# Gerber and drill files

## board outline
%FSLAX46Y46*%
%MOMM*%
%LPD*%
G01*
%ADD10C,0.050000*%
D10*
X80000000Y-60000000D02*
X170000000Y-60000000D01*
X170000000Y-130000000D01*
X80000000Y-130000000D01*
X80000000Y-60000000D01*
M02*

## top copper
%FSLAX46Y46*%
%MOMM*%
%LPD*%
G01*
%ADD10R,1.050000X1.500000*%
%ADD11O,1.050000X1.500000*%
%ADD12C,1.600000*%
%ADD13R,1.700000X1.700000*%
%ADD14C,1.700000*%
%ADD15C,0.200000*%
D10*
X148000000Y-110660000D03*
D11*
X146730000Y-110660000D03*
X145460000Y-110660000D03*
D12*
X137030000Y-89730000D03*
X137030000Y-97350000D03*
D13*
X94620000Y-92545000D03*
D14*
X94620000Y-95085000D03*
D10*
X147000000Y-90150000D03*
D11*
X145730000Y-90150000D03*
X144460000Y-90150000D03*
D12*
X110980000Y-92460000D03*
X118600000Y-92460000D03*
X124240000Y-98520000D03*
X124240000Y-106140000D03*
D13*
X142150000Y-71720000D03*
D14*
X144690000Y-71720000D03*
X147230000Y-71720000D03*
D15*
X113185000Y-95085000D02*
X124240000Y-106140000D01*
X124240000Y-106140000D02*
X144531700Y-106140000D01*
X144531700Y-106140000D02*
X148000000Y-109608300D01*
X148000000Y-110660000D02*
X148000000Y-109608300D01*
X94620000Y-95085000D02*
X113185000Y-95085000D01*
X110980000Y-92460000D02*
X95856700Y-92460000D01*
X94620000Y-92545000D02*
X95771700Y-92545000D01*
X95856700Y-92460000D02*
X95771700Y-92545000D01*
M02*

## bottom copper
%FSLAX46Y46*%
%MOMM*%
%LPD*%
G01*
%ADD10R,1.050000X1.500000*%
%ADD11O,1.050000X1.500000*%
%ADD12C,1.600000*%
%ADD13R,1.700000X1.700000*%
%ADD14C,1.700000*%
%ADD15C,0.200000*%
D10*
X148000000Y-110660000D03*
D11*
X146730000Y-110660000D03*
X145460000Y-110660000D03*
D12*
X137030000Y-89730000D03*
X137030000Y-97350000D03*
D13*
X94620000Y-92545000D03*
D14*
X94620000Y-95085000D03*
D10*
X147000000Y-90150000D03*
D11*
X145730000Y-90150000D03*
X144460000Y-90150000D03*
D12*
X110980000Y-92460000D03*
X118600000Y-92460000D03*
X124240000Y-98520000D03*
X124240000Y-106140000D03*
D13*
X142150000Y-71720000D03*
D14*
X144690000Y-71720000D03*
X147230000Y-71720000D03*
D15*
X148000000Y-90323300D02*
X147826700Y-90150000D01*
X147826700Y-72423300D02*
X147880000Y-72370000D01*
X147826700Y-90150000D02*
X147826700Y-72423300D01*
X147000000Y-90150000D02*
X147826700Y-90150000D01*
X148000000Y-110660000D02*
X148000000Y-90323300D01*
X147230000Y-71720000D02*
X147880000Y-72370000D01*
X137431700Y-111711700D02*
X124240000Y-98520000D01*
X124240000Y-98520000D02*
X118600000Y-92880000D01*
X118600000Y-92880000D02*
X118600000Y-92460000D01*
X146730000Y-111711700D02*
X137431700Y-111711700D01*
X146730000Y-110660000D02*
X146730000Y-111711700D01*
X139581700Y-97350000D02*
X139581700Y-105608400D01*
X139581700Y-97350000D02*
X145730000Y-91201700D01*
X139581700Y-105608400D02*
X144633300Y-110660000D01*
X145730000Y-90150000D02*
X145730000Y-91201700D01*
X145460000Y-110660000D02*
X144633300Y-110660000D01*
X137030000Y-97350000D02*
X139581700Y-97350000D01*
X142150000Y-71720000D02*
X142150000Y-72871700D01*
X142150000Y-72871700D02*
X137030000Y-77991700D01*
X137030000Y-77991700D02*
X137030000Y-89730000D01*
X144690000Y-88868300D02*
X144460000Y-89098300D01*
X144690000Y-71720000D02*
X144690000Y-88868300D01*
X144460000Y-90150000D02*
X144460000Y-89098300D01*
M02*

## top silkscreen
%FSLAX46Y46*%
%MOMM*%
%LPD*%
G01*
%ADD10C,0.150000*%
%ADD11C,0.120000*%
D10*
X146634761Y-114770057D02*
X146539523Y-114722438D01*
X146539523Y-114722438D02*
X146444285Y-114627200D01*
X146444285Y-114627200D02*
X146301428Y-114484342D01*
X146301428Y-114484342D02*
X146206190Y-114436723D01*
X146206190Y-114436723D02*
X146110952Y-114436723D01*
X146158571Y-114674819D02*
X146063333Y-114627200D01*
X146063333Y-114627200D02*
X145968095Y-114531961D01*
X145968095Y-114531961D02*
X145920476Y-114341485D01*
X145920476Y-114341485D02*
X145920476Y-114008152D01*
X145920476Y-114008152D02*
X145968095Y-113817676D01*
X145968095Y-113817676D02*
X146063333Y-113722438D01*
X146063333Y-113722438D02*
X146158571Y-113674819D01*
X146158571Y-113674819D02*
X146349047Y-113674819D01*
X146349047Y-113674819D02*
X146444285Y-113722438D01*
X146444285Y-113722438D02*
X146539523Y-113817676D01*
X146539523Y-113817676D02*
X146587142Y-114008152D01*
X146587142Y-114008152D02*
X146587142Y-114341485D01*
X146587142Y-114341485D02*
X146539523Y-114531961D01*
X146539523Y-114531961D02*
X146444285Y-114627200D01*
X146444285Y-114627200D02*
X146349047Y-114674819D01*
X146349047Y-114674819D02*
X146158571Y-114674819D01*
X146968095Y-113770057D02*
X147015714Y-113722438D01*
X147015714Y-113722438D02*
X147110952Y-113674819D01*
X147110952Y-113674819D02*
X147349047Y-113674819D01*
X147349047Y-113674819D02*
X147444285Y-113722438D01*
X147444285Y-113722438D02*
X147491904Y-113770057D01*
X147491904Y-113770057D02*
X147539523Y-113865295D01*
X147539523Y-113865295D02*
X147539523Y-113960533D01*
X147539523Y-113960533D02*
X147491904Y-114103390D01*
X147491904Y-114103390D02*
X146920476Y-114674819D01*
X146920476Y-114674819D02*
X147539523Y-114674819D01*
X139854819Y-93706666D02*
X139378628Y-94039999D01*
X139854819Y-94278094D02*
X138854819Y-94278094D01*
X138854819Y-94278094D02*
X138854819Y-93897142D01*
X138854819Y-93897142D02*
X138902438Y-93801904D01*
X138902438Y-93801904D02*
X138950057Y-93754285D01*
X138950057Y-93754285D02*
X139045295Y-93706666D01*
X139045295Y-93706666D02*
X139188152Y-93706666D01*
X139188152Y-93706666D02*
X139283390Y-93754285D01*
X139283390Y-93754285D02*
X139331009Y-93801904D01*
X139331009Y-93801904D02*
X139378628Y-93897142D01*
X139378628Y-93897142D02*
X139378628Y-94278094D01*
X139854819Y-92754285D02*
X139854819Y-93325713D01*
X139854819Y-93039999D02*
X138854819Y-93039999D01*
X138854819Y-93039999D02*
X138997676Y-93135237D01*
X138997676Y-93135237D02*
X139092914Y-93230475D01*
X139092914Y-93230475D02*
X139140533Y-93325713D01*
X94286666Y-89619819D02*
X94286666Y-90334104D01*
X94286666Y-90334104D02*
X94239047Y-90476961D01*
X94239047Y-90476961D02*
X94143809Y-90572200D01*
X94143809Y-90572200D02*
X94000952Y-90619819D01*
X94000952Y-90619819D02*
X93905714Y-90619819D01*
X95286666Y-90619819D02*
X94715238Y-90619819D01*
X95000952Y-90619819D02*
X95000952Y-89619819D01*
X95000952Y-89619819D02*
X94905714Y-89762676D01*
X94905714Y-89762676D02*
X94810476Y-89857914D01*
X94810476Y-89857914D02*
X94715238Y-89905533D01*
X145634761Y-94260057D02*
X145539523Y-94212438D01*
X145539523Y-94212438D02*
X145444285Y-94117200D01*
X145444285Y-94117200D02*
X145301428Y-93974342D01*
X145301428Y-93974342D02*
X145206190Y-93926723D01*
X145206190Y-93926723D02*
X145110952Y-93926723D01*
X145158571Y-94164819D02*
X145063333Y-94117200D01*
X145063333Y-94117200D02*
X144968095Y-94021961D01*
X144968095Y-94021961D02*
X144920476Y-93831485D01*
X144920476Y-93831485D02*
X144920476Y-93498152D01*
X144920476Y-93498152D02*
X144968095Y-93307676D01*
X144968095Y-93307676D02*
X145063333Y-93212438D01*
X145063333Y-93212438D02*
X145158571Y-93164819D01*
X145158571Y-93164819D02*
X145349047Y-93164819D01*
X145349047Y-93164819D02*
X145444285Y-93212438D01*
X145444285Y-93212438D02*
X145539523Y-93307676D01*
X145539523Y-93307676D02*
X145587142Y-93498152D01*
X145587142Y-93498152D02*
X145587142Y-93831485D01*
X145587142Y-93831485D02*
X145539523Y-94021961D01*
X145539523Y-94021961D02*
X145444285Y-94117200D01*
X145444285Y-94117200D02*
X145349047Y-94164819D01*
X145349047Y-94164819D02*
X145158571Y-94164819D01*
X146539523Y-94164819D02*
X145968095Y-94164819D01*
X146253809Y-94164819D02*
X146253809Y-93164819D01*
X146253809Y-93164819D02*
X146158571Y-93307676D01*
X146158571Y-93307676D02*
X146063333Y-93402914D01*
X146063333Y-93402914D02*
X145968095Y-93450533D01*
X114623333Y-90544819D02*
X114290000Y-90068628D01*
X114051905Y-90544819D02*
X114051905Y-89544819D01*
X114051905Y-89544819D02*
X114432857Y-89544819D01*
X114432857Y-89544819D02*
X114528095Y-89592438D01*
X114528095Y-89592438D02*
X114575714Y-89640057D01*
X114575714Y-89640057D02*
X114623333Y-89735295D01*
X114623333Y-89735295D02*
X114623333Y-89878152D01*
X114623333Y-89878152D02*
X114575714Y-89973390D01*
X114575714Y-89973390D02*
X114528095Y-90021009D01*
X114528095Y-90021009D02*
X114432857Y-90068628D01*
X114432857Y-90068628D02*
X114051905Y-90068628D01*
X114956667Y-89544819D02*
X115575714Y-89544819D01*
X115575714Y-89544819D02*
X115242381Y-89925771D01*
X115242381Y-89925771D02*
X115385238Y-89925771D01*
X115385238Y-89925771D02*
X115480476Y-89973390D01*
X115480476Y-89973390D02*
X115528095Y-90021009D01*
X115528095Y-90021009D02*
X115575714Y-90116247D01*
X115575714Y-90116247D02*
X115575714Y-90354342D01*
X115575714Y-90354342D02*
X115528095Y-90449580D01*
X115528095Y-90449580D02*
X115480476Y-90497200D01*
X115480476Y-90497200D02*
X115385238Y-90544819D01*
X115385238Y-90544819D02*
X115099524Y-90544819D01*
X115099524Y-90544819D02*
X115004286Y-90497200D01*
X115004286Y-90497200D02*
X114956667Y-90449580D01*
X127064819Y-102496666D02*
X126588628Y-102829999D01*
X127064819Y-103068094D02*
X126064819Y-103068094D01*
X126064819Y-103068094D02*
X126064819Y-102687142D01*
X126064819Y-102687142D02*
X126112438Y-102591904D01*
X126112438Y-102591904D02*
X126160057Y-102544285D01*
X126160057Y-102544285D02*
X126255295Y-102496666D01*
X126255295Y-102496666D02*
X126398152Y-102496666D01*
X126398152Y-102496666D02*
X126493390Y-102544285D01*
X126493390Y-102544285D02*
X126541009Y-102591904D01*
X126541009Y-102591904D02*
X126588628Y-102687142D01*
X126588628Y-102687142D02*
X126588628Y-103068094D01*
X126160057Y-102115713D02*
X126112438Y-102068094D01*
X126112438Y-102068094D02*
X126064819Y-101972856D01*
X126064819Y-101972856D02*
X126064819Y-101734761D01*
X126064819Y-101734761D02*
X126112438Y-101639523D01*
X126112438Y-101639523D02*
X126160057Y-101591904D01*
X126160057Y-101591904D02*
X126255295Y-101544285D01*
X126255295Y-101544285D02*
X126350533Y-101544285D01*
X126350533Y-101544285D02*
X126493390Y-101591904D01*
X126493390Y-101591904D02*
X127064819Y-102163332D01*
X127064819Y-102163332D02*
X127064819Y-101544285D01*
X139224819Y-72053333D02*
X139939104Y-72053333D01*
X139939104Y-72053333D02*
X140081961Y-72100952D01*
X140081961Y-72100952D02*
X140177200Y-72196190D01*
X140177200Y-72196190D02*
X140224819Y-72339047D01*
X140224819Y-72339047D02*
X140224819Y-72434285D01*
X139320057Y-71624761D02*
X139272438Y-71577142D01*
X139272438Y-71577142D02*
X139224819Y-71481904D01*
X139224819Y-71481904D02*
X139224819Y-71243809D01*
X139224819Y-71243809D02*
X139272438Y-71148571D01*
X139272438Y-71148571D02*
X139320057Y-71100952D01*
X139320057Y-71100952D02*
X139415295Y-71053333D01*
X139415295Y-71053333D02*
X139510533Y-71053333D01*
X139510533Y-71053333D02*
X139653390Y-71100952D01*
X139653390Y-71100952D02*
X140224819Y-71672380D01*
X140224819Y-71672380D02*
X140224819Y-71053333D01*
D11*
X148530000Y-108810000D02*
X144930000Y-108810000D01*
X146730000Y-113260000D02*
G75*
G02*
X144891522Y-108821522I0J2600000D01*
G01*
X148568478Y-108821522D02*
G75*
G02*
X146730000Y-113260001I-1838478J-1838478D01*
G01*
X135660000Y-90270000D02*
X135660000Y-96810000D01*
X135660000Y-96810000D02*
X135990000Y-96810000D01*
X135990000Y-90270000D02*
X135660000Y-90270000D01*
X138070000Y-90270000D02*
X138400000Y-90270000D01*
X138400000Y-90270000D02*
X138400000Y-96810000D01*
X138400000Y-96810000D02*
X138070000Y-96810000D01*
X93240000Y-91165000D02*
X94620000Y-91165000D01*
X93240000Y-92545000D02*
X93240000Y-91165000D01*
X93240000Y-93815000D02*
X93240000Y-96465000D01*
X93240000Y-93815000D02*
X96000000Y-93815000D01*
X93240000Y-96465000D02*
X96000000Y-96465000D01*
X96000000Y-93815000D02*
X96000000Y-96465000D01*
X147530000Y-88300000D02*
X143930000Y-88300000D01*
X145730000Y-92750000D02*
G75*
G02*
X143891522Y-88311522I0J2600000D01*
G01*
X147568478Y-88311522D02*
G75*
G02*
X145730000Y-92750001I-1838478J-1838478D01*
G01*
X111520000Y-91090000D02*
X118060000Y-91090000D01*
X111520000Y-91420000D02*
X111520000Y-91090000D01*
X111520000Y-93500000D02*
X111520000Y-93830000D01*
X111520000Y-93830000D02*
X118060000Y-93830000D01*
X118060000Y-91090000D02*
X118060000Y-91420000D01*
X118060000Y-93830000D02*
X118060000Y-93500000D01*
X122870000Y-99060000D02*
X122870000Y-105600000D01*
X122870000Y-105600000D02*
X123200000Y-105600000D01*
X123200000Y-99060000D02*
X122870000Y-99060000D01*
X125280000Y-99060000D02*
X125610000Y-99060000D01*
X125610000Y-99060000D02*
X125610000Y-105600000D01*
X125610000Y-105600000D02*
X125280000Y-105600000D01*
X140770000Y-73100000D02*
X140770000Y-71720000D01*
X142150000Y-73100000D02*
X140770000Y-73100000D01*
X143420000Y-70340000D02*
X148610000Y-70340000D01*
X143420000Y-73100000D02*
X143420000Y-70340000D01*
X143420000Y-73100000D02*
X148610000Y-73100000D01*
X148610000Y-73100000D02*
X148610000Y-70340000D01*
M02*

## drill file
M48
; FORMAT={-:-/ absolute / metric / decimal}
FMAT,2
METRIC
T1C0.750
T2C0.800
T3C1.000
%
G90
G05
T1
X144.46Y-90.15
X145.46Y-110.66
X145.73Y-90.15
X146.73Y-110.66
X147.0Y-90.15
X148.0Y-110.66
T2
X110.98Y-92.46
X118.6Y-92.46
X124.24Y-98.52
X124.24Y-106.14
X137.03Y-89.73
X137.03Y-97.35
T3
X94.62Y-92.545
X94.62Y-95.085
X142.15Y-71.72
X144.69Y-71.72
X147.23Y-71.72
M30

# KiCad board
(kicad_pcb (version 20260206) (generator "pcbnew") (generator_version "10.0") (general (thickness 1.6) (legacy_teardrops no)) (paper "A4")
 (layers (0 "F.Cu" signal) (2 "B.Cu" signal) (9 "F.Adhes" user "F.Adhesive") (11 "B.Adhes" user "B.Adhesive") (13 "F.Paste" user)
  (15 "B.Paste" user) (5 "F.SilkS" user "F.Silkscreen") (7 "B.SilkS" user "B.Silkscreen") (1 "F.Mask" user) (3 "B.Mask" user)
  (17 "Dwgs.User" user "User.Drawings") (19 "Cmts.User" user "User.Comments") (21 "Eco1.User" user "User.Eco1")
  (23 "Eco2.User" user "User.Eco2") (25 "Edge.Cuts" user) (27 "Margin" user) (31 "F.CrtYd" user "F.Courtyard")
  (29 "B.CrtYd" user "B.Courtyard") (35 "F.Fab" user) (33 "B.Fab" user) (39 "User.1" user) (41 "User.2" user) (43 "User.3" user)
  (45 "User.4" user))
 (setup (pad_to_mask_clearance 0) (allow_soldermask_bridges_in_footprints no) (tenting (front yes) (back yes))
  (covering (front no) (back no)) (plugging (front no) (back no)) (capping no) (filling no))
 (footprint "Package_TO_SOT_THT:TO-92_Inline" (layer "F.Cu") (at 148 110.66 180)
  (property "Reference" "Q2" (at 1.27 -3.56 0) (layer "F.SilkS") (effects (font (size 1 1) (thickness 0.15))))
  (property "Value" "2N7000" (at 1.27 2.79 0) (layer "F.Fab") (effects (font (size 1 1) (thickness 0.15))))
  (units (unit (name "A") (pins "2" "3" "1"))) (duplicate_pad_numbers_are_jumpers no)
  (fp_line (start -0.53 1.85) (end 3.07 1.85) (stroke (width 0.12) (type solid)) (layer "F.SilkS"))
  (fp_arc (start 1.27 -2.6) (mid 3.672087 -0.994977) (end 3.108478 1.838478) (stroke (width 0.12) (type solid)) (layer "F.SilkS"))
  (fp_arc (start -0.568478 1.838478) (mid -1.132087 -0.994977) (end 1.27 -2.6) (stroke (width 0.12) (type solid)) (layer "F.SilkS"))
  (pad "1" thru_hole rect (at 0 0 180) (size 1.05 1.5) (drill 0.75) (layers "*.Cu" "*.Mask") (remove_unused_layers no) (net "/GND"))
  (pad "2" thru_hole oval (at 1.27 0 180) (size 1.05 1.5) (drill 0.75) (layers "*.Cu" "*.Mask") (remove_unused_layers no) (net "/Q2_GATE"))
  (pad "3" thru_hole oval (at 2.54 0 180) (size 1.05 1.5) (drill 0.75) (layers "*.Cu" "*.Mask") (remove_unused_layers no) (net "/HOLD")))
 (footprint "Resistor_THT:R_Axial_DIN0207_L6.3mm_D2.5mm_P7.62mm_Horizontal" (layer "F.Cu") (at 137.03 89.73 -90)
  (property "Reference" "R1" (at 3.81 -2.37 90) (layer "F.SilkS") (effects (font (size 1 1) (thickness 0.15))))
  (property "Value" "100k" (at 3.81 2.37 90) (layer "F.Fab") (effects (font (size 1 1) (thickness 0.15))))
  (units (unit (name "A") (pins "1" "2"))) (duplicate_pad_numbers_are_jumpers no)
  (fp_line (start 0.54 1.37) (end 7.08 1.37) (stroke (width 0.12) (type solid)) (layer "F.SilkS"))
  (fp_line (start 7.08 1.37) (end 7.08 1.04) (stroke (width 0.12) (type solid)) (layer "F.SilkS"))
  (fp_line (start 0.54 1.04) (end 0.54 1.37) (stroke (width 0.12) (type solid)) (layer "F.SilkS"))
  (fp_line (start 0.54 -1.04) (end 0.54 -1.37) (stroke (width 0.12) (type solid)) (layer "F.SilkS"))
  (fp_line (start 0.54 -1.37) (end 7.08 -1.37) (stroke (width 0.12) (type solid)) (layer "F.SilkS"))
  (fp_line (start 7.08 -1.37) (end 7.08 -1.04) (stroke (width 0.12) (type solid)) (layer "F.SilkS"))
  (pad "1" thru_hole circle (at 0 0 270) (size 1.6 1.6) (drill 0.8) (layers "*.Cu" "*.Mask") (remove_unused_layers no) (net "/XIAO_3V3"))
  (pad "2" thru_hole circle (at 7.62 0 270) (size 1.6 1.6) (drill 0.8) (layers "*.Cu" "*.Mask") (remove_unused_layers no) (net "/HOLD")))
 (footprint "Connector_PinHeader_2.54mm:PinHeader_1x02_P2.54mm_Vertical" (layer "F.Cu") (at 94.62 92.545)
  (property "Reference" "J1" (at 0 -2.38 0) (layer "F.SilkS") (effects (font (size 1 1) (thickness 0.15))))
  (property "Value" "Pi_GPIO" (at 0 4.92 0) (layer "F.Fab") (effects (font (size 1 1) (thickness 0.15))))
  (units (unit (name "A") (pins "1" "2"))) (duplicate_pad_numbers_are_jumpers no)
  (fp_line (start -1.38 -1.38) (end 0 -1.38) (stroke (width 0.12) (type solid)) (layer "F.SilkS"))
  (fp_line (start -1.38 0) (end -1.38 -1.38) (stroke (width 0.12) (type solid)) (layer "F.SilkS"))
  (fp_line (start -1.38 1.27) (end -1.38 3.92) (stroke (width 0.12) (type solid)) (layer "F.SilkS"))
  (fp_line (start -1.38 1.27) (end 1.38 1.27) (stroke (width 0.12) (type solid)) (layer "F.SilkS"))
  (fp_line (start -1.38 3.92) (end 1.38 3.92) (stroke (width 0.12) (type solid)) (layer "F.SilkS"))
  (fp_line (start 1.38 1.27) (end 1.38 3.92) (stroke (width 0.12) (type solid)) (layer "F.SilkS"))
  (pad "1" thru_hole rect (at 0 0) (size 1.7 1.7) (drill 1) (layers "*.Cu" "*.Mask") (remove_unused_layers no) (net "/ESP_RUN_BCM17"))
  (pad "2" thru_hole circle (at 0 2.54) (size 1.7 1.7) (drill 1) (layers "*.Cu" "*.Mask") (remove_unused_layers no) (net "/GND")))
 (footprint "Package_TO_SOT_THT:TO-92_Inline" (layer "F.Cu") (at 147 90.15 180)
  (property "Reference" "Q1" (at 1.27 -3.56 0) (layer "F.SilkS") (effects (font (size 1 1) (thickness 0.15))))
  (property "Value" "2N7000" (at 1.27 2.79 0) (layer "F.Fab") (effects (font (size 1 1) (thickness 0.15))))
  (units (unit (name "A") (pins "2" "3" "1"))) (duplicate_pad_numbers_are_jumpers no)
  (fp_line (start -0.53 1.85) (end 3.07 1.85) (stroke (width 0.12) (type solid)) (layer "F.SilkS"))
  (fp_arc (start 1.27 -2.6) (mid 3.672087 -0.994977) (end 3.108478 1.838478) (stroke (width 0.12) (type solid)) (layer "F.SilkS"))
  (fp_arc (start -0.568478 1.838478) (mid -1.132087 -0.994977) (end 1.27 -2.6) (stroke (width 0.12) (type solid)) (layer "F.SilkS"))
  (pad "1" thru_hole rect (at 0 0 180) (size 1.05 1.5) (drill 0.75) (layers "*.Cu" "*.Mask") (remove_unused_layers no) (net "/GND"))
  (pad "2" thru_hole oval (at 1.27 0 180) (size 1.05 1.5) (drill 0.75) (layers "*.Cu" "*.Mask") (remove_unused_layers no) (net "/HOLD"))
  (pad "3" thru_hole oval (at 2.54 0 180) (size 1.05 1.5) (drill 0.75) (layers "*.Cu" "*.Mask") (remove_unused_layers no)
   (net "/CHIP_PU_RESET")))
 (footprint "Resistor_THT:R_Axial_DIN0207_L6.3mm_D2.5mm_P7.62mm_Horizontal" (layer "F.Cu") (at 110.98 92.46)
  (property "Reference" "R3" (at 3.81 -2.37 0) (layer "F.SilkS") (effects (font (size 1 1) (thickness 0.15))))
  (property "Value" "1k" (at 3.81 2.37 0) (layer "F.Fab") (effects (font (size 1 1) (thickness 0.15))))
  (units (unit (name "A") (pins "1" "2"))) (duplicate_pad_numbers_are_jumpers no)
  (fp_line (start 0.54 -1.37) (end 7.08 -1.37) (stroke (width 0.12) (type solid)) (layer "F.SilkS"))
  (fp_line (start 0.54 -1.04) (end 0.54 -1.37) (stroke (width 0.12) (type solid)) (layer "F.SilkS"))
  (fp_line (start 0.54 1.04) (end 0.54 1.37) (stroke (width 0.12) (type solid)) (layer "F.SilkS"))
  (fp_line (start 0.54 1.37) (end 7.08 1.37) (stroke (width 0.12) (type solid)) (layer "F.SilkS"))
  (fp_line (start 7.08 -1.37) (end 7.08 -1.04) (stroke (width 0.12) (type solid)) (layer "F.SilkS"))
  (fp_line (start 7.08 1.37) (end 7.08 1.04) (stroke (width 0.12) (type solid)) (layer "F.SilkS"))
  (pad "1" thru_hole circle (at 0 0) (size 1.6 1.6) (drill 0.8) (layers "*.Cu" "*.Mask") (remove_unused_layers no) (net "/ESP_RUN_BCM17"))
  (pad "2" thru_hole circle (at 7.62 0) (size 1.6 1.6) (drill 0.8) (layers "*.Cu" "*.Mask") (remove_unused_layers no) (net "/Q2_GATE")))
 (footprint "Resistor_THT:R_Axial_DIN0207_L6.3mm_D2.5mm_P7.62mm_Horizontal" (layer "F.Cu") (at 124.24 98.52 -90)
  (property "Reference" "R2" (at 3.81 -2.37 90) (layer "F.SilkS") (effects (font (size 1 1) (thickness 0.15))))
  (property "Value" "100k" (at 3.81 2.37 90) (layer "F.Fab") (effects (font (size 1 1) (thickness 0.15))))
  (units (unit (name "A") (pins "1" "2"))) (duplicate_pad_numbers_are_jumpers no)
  (fp_line (start 0.54 1.37) (end 7.08 1.37) (stroke (width 0.12) (type solid)) (layer "F.SilkS"))
  (fp_line (start 7.08 1.37) (end 7.08 1.04) (stroke (width 0.12) (type solid)) (layer "F.SilkS"))
  (fp_line (start 0.54 1.04) (end 0.54 1.37) (stroke (width 0.12) (type solid)) (layer "F.SilkS"))
  (fp_line (start 0.54 -1.04) (end 0.54 -1.37) (stroke (width 0.12) (type solid)) (layer "F.SilkS"))
  (fp_line (start 0.54 -1.37) (end 7.08 -1.37) (stroke (width 0.12) (type solid)) (layer "F.SilkS"))
  (fp_line (start 7.08 -1.37) (end 7.08 -1.04) (stroke (width 0.12) (type solid)) (layer "F.SilkS"))
  (pad "1" thru_hole circle (at 0 0 270) (size 1.6 1.6) (drill 0.8) (layers "*.Cu" "*.Mask") (remove_unused_layers no) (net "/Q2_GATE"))
  (pad "2" thru_hole circle (at 7.62 0 270) (size 1.6 1.6) (drill 0.8) (layers "*.Cu" "*.Mask") (remove_unused_layers no) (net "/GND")))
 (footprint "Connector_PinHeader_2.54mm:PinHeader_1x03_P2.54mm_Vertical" (layer "F.Cu") (at 142.15 71.72 90)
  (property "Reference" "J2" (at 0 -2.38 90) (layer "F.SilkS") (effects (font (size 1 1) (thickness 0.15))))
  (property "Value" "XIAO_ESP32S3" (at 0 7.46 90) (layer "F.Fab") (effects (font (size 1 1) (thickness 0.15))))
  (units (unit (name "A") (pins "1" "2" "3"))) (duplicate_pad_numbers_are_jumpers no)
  (fp_line (start -1.38 -1.38) (end 0 -1.38) (stroke (width 0.12) (type solid)) (layer "F.SilkS"))
  (fp_line (start -1.38 0) (end -1.38 -1.38) (stroke (width 0.12) (type solid)) (layer "F.SilkS"))
  (fp_line (start 1.38 1.27) (end 1.38 6.46) (stroke (width 0.12) (type solid)) (layer "F.SilkS"))
  (fp_line (start -1.38 1.27) (end 1.38 1.27) (stroke (width 0.12) (type solid)) (layer "F.SilkS"))
  (fp_line (start -1.38 1.27) (end -1.38 6.46) (stroke (width 0.12) (type solid)) (layer "F.SilkS"))
  (fp_line (start -1.38 6.46) (end 1.38 6.46) (stroke (width 0.12) (type solid)) (layer "F.SilkS"))
  (pad "1" thru_hole rect (at 0 0 90) (size 1.7 1.7) (drill 1) (layers "*.Cu" "*.Mask") (remove_unused_layers no) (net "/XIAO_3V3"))
  (pad "2" thru_hole circle (at 0 2.54 90) (size 1.7 1.7) (drill 1) (layers "*.Cu" "*.Mask") (remove_unused_layers no)
   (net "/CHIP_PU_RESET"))
  (pad "3" thru_hole circle (at 0 5.08 90) (size 1.7 1.7) (drill 1) (layers "*.Cu" "*.Mask") (remove_unused_layers no) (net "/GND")))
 (gr_rect (start 80 60) (end 170 130) (stroke (width 0.05) (type solid)) (fill no) (layer "Edge.Cuts"))
 (segment (start 113.185 95.085) (end 124.24 106.14) (width 0.2) (layer "F.Cu") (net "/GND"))
 (segment (start 124.24 106.14) (end 144.5317 106.14) (width 0.2) (layer "F.Cu") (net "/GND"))
 (segment (start 144.5317 106.14) (end 148 109.6083) (width 0.2) (layer "F.Cu") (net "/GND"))
 (segment (start 148 110.66) (end 148 109.6083) (width 0.2) (layer "F.Cu") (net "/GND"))
 (segment (start 94.62 95.085) (end 113.185 95.085) (width 0.2) (layer "F.Cu") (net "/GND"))
 (segment (start 148 90.3233) (end 147.8267 90.15) (width 0.2) (layer "B.Cu") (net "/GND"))
 (segment (start 147.8267 72.4233) (end 147.88 72.37) (width 0.2) (layer "B.Cu") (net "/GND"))
 (segment (start 147.8267 90.15) (end 147.8267 72.4233) (width 0.2) (layer "B.Cu") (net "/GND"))
 (segment (start 147 90.15) (end 147.8267 90.15) (width 0.2) (layer "B.Cu") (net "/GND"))
 (segment (start 148 110.66) (end 148 90.3233) (width 0.2) (layer "B.Cu") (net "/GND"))
 (segment (start 147.23 71.72) (end 147.88 72.37) (width 0.2) (layer "B.Cu") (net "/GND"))
 (segment (start 137.4317 111.7117) (end 124.24 98.52) (width 0.2) (layer "B.Cu") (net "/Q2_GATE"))
 (segment (start 124.24 98.52) (end 118.6 92.88) (width 0.2) (layer "B.Cu") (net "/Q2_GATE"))
 (segment (start 118.6 92.88) (end 118.6 92.46) (width 0.2) (layer "B.Cu") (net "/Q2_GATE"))
 (segment (start 146.73 111.7117) (end 137.4317 111.7117) (width 0.2) (layer "B.Cu") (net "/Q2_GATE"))
 (segment (start 146.73 110.66) (end 146.73 111.7117) (width 0.2) (layer "B.Cu") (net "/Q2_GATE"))
 (segment (start 139.5817 97.35) (end 139.5817 105.6084) (width 0.2) (layer "B.Cu") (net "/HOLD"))
 (segment (start 139.5817 97.35) (end 145.73 91.2017) (width 0.2) (layer "B.Cu") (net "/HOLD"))
 (segment (start 139.5817 105.6084) (end 144.6333 110.66) (width 0.2) (layer "B.Cu") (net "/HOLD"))
 (segment (start 145.73 90.15) (end 145.73 91.2017) (width 0.2) (layer "B.Cu") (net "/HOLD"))
 (segment (start 145.46 110.66) (end 144.6333 110.66) (width 0.2) (layer "B.Cu") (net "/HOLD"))
 (segment (start 137.03 97.35) (end 139.5817 97.35) (width 0.2) (layer "B.Cu") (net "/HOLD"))
 (segment (start 142.15 71.72) (end 142.15 72.8717) (width 0.2) (layer "B.Cu") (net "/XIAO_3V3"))
 (segment (start 142.15 72.8717) (end 137.03 77.9917) (width 0.2) (layer "B.Cu") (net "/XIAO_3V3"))
 (segment (start 137.03 77.9917) (end 137.03 89.73) (width 0.2) (layer "B.Cu") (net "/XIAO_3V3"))
 (segment (start 110.98 92.46) (end 95.8567 92.46) (width 0.2) (layer "F.Cu") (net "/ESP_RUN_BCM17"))
 (segment (start 94.62 92.545) (end 95.7717 92.545) (width 0.2) (layer "F.Cu") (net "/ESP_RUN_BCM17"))
 (segment (start 95.8567 92.46) (end 95.7717 92.545) (width 0.2) (layer "F.Cu") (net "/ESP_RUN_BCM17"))
 (segment (start 144.69 88.8683) (end 144.46 89.0983) (width 0.2) (layer "B.Cu") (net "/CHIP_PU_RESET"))
 (segment (start 144.69 71.72) (end 144.69 88.8683) (width 0.2) (layer "B.Cu") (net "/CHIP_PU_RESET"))
 (segment (start 144.46 90.15) (end 144.46 89.0983) (width 0.2) (layer "B.Cu") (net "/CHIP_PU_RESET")))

